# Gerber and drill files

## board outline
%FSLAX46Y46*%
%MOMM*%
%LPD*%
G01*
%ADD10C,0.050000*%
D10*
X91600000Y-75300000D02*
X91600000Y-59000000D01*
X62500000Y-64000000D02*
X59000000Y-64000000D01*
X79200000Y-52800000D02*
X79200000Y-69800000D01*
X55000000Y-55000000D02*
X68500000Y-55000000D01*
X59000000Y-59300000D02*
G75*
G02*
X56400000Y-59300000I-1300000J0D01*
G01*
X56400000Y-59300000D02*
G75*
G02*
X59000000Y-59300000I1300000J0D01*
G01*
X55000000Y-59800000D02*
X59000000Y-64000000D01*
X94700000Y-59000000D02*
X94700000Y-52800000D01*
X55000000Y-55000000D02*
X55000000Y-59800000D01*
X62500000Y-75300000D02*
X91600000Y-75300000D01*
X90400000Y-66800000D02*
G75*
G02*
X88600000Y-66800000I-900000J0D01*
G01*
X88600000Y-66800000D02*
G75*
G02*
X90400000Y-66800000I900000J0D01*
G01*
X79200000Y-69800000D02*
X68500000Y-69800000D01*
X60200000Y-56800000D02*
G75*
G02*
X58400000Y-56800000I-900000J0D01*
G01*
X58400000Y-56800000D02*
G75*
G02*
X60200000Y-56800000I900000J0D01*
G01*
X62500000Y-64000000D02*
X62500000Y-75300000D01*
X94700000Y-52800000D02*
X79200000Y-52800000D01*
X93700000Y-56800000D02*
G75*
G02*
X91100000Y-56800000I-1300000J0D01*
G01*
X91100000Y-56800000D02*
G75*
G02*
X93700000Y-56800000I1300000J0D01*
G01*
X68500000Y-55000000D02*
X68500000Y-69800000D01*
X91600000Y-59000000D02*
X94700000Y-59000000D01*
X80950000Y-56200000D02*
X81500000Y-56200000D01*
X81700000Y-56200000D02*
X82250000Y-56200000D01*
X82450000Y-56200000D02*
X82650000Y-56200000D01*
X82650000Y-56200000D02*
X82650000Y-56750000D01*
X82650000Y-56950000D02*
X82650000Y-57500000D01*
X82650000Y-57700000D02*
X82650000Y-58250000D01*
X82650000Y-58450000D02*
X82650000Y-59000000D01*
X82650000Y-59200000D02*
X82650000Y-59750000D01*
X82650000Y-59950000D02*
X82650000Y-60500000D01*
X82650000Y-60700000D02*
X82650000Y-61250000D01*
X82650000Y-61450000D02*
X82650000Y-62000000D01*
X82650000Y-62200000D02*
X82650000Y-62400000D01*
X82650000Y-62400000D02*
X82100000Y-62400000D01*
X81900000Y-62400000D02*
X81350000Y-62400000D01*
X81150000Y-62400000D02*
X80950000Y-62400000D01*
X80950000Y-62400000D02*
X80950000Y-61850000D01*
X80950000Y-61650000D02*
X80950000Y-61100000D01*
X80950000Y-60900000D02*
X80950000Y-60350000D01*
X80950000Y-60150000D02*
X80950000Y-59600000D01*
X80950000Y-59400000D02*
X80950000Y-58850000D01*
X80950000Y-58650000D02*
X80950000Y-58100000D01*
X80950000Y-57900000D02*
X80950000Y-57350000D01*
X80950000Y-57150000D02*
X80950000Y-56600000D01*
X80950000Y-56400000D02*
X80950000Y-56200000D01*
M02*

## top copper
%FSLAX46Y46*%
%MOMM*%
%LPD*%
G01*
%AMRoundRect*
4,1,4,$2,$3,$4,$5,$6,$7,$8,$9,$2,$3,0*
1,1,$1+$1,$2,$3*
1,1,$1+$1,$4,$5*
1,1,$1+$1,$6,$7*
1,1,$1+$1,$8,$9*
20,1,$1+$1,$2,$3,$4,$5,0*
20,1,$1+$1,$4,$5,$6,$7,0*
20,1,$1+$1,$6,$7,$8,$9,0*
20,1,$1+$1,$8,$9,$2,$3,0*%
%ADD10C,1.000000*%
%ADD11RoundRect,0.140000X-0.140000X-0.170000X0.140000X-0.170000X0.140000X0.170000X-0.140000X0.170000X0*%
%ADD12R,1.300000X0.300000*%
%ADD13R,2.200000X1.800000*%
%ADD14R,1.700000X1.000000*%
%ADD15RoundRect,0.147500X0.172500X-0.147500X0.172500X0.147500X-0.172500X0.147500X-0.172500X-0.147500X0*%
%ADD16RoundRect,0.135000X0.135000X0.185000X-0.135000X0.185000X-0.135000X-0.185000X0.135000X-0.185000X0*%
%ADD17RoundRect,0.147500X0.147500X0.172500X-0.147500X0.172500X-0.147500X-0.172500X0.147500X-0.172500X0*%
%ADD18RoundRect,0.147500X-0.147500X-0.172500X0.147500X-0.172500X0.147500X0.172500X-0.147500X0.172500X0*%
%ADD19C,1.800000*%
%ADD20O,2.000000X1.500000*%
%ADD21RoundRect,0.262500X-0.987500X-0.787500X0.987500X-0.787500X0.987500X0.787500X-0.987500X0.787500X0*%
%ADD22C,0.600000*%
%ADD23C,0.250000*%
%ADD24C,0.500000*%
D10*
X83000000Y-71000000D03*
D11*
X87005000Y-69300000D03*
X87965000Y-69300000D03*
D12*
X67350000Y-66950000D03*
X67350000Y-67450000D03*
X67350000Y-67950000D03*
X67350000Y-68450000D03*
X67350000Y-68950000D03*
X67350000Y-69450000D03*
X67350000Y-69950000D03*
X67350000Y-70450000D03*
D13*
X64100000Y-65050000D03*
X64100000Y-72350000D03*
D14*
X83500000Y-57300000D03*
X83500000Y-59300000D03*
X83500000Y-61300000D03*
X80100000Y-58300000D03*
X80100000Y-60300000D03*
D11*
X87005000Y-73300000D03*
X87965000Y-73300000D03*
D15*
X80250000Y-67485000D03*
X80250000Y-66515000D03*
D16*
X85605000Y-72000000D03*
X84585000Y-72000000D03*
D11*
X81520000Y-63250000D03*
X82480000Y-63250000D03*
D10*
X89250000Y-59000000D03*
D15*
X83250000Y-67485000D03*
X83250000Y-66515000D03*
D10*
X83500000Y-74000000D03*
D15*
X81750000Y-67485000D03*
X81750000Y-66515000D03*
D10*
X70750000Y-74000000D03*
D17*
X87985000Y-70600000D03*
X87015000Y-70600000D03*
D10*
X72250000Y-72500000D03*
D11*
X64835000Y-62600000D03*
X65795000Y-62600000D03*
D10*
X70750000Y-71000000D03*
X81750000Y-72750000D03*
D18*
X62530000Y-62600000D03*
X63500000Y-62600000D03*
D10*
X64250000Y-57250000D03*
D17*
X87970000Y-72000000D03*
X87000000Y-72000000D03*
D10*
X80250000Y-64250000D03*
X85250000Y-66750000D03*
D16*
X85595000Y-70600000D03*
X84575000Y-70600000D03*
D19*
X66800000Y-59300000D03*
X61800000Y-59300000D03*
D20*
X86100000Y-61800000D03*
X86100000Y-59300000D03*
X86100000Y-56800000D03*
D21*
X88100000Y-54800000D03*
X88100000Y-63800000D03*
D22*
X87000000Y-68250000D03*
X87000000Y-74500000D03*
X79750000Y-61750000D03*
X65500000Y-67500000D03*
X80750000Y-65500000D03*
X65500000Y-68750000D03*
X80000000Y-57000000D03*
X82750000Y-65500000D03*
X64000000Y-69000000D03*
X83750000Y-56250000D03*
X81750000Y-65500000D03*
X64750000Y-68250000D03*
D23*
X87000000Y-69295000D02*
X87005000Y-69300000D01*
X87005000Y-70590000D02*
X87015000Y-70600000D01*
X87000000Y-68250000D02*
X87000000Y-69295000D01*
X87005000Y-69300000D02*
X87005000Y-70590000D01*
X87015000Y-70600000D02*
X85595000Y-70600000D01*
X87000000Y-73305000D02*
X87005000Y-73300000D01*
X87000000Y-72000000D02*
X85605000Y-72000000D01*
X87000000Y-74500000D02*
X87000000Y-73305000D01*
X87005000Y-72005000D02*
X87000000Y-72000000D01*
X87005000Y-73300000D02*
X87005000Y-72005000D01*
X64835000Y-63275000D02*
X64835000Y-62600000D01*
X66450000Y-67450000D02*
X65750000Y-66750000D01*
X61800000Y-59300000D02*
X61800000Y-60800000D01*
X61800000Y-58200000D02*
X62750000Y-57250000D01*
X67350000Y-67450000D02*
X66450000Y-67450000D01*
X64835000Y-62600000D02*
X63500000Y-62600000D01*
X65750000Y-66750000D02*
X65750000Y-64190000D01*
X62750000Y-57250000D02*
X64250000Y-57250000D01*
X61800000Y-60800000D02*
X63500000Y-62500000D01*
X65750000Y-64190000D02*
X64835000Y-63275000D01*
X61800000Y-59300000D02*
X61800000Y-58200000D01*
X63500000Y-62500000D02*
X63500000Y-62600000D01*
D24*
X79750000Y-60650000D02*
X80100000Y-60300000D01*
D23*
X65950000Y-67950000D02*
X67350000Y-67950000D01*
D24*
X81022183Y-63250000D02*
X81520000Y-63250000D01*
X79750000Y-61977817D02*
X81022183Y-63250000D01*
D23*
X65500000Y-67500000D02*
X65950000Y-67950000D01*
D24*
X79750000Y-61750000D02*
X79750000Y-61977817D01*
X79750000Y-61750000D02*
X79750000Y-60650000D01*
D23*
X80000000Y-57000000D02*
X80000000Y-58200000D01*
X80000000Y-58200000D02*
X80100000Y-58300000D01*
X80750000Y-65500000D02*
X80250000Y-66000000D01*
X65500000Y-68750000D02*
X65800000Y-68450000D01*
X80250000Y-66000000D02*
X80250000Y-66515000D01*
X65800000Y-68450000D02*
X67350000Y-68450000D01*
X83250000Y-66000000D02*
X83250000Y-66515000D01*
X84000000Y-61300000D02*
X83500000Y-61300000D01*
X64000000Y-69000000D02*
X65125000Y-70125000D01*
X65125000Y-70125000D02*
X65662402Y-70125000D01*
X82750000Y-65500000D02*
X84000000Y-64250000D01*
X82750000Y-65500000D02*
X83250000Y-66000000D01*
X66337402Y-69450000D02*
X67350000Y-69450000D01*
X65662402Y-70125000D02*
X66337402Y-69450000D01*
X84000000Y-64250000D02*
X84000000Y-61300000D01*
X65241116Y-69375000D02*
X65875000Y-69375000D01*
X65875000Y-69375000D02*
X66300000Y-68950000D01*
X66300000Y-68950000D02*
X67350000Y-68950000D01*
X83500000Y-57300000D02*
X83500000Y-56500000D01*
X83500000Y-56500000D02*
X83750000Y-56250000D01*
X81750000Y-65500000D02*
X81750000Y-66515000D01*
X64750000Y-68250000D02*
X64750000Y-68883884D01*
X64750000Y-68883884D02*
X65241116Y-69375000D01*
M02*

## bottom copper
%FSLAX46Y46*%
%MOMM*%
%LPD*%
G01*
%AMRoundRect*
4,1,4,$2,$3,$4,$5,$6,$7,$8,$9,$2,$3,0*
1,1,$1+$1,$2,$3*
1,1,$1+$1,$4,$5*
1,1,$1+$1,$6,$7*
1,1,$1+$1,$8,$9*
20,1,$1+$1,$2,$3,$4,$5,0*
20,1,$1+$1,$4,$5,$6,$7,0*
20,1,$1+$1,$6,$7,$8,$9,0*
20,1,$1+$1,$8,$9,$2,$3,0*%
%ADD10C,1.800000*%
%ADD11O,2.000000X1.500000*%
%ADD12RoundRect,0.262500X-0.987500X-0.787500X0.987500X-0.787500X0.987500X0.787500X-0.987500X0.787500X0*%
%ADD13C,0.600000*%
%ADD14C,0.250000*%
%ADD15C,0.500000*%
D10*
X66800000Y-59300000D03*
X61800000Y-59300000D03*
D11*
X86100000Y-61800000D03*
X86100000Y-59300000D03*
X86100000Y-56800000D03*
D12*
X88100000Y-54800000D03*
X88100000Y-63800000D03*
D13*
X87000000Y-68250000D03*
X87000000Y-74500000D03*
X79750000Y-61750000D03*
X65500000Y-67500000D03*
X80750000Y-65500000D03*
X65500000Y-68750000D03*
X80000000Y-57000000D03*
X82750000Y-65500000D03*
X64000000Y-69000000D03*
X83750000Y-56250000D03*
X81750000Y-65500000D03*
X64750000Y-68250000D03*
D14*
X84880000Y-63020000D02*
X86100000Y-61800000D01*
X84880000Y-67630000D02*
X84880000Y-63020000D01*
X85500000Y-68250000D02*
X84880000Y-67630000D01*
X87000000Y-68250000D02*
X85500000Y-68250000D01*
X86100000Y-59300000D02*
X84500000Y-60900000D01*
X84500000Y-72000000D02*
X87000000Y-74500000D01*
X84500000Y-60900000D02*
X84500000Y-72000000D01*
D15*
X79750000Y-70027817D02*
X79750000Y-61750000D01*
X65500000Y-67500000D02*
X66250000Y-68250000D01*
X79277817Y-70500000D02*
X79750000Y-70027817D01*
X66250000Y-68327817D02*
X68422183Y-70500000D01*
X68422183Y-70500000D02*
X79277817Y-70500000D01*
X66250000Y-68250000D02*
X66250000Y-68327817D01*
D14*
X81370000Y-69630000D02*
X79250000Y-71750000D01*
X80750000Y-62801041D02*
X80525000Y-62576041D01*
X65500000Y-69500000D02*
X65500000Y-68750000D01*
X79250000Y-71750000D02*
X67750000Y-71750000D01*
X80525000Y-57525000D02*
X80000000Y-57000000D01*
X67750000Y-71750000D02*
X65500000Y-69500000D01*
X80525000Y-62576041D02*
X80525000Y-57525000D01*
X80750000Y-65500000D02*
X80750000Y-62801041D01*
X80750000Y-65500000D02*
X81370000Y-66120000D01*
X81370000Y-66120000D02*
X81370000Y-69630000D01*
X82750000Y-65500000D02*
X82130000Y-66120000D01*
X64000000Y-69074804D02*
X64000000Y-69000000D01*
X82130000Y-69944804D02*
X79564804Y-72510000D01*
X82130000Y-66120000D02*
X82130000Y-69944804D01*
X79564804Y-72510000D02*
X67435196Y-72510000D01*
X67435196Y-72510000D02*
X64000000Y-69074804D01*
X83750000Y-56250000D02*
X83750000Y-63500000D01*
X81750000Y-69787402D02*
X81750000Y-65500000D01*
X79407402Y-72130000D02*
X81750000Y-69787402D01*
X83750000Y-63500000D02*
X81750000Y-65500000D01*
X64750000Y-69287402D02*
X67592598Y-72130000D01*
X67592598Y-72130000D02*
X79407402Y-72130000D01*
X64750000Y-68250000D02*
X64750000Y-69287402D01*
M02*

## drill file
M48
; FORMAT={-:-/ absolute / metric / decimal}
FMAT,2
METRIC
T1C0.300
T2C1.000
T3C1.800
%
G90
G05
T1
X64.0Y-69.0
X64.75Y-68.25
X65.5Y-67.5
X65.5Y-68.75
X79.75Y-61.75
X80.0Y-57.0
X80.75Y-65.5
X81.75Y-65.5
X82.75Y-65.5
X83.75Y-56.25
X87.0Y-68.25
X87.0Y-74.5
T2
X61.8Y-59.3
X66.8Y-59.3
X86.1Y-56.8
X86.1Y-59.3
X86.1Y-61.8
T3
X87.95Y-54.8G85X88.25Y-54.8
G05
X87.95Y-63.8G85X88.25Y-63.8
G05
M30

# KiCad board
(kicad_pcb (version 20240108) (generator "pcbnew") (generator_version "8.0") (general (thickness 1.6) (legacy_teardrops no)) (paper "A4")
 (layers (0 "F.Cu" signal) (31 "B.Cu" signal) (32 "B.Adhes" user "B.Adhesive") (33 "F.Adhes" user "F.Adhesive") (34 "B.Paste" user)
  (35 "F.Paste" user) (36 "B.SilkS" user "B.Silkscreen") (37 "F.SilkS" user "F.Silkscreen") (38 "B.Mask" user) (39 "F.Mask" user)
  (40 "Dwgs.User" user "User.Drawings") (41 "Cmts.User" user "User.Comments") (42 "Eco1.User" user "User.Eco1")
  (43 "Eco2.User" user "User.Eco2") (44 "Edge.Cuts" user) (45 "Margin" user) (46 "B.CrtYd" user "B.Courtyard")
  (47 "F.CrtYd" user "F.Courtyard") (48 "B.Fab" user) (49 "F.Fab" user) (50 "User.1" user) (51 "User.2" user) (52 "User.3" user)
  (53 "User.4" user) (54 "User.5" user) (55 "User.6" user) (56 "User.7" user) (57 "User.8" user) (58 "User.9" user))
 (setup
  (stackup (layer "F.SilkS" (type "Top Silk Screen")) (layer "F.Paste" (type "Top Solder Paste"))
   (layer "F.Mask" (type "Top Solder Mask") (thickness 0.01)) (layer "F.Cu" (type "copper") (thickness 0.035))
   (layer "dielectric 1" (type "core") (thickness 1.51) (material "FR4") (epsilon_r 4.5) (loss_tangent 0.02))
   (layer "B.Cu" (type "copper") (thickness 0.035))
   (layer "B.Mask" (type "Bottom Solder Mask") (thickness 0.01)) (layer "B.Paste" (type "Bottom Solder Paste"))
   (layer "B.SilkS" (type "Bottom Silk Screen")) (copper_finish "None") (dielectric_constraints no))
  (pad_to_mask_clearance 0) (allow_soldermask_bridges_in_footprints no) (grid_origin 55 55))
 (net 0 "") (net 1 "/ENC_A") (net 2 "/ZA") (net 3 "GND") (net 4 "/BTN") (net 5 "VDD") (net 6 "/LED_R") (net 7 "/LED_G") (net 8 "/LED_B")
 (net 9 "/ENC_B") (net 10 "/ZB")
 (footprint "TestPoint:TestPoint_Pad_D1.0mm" (layer "F.Cu") (at 83 71)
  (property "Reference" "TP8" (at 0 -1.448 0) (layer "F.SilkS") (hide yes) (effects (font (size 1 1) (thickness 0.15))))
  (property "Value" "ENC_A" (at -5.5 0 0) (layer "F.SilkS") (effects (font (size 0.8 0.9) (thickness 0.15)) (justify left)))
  (pad "1" smd circle (at 0 0) (size 1 1) (layers "F.Cu" "F.Mask") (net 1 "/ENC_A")))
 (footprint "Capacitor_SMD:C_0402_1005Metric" (layer "F.Cu") (at 87.485 69.3)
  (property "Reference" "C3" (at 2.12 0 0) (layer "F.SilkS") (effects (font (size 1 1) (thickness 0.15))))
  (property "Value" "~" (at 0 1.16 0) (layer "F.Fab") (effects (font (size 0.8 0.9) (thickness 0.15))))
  (pad "1" smd roundrect (at -0.48 0) (size 0.56 0.62) (layers "F.Cu" "F.Paste" "F.Mask") (roundrect_rratio 0.25) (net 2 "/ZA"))
  (pad "2" smd roundrect (at 0.48 0) (size 0.56 0.62) (layers "F.Cu" "F.Paste" "F.Mask") (roundrect_rratio 0.25) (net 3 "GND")))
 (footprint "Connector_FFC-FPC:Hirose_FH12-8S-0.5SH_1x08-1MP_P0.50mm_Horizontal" (layer "F.Cu") (at 65.5 68.7 -90)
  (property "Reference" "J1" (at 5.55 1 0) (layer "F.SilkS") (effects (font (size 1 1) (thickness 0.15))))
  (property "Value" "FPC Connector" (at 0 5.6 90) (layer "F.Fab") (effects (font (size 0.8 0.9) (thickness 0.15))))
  (pad "1" smd rect (at -1.75 -1.85 270) (size 0.3 1.3) (layers "F.Cu" "F.Paste" "F.Mask") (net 3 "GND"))
  (pad "2" smd rect (at -1.25 -1.85 270) (size 0.3 1.3) (layers "F.Cu" "F.Paste" "F.Mask") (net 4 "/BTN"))
  (pad "3" smd rect (at -0.75 -1.85 270) (size 0.3 1.3) (layers "F.Cu" "F.Paste" "F.Mask") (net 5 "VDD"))
  (pad "4" smd rect (at -0.25 -1.85 270) (size 0.3 1.3) (layers "F.Cu" "F.Paste" "F.Mask") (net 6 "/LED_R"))
  (pad "5" smd rect (at 0.25 -1.85 270) (size 0.3 1.3) (layers "F.Cu" "F.Paste" "F.Mask") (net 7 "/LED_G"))
  (pad "6" smd rect (at 0.75 -1.85 270) (size 0.3 1.3) (layers "F.Cu" "F.Paste" "F.Mask") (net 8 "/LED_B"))
  (pad "7" smd rect (at 1.25 -1.85 270) (size 0.3 1.3) (layers "F.Cu" "F.Paste" "F.Mask") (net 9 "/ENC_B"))
  (pad "8" smd rect (at 1.75 -1.85 270) (size 0.3 1.3) (layers "F.Cu" "F.Paste" "F.Mask") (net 1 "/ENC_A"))
  (pad "MP" smd rect (at -3.65 1.4 270) (size 1.8 2.2) (layers "F.Cu" "F.Paste" "F.Mask") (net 3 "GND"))
  (pad "MP" smd rect (at 3.65 1.4 270) (size 1.8 2.2) (layers "F.Cu" "F.Paste" "F.Mask") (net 3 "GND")))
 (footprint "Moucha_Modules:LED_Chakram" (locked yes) (layer "F.Cu") (at 81.8 59.3)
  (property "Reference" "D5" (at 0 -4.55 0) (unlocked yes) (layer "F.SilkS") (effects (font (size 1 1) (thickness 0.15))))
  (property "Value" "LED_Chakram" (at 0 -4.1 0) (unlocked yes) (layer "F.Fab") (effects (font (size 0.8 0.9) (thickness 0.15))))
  (fp_rect (start -0.85 -3.1) (end 0.85 3.1) (stroke (width 0.05) (type dash)) (fill none) (layer "Edge.Cuts"))
  (pad "1" smd rect (at 1.7 -2) (size 1.7 1) (layers "F.Cu" "F.Paste" "F.Mask") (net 7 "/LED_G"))
  (pad "2" smd rect (at 1.7 0) (size 1.7 1) (layers "F.Cu" "F.Paste" "F.Mask") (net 3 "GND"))
  (pad "3" smd rect (at 1.7 2) (size 1.7 1) (layers "F.Cu" "F.Paste" "F.Mask") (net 8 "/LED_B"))
  (pad "4" smd rect (at -1.7 -1) (size 1.7 1) (layers "F.Cu" "F.Paste" "F.Mask") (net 6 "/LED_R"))
  (pad "5" smd rect (at -1.7 1) (size 1.7 1) (layers "F.Cu" "F.Paste" "F.Mask") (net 5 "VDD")))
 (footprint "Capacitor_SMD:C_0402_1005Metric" (layer "F.Cu") (at 87.485 73.3)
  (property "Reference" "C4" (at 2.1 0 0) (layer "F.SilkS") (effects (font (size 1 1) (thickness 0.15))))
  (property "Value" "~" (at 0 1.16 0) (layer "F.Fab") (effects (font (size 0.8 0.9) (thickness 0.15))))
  (pad "1" smd roundrect (at -0.48 0) (size 0.56 0.62) (layers "F.Cu" "F.Paste" "F.Mask") (roundrect_rratio 0.25) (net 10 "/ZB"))
  (pad "2" smd roundrect (at 0.48 0) (size 0.56 0.62) (layers "F.Cu" "F.Paste" "F.Mask") (roundrect_rratio 0.25) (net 3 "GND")))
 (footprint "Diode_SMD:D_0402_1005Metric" (layer "F.Cu") (at 80.25 67 90)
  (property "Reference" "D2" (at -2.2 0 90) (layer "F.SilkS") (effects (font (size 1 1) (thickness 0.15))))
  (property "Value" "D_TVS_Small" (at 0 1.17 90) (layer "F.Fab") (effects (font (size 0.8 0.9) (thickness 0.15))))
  (pad "1" smd roundrect (at -0.485 0 90) (size 0.59 0.64) (layers "F.Cu" "F.Paste" "F.Mask") (roundrect_rratio 0.25) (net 3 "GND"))
  (pad "2" smd roundrect (at 0.485 0 90) (size 0.59 0.64) (layers "F.Cu" "F.Paste" "F.Mask") (roundrect_rratio 0.25) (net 6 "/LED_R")))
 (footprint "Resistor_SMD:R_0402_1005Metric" (layer "F.Cu") (at 85.095 72 180)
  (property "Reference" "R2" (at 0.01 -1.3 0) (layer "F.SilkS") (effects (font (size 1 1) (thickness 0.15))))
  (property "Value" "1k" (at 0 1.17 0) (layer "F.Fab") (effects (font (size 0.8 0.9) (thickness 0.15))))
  (pad "1" smd roundrect (at -0.51 0 180) (size 0.54 0.64) (layers "F.Cu" "F.Paste" "F.Mask") (roundrect_rratio 0.25) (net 10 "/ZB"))
  (pad "2" smd roundrect (at 0.51 0 180) (size 0.54 0.64) (layers "F.Cu" "F.Paste" "F.Mask") (roundrect_rratio 0.25) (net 9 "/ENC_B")))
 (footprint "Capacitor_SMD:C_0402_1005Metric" (layer "F.Cu") (at 82 63.25)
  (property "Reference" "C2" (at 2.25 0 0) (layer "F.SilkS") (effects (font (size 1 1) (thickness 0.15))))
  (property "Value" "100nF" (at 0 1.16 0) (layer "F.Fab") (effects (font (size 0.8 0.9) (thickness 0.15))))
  (pad "1" smd roundrect (at -0.48 0) (size 0.56 0.62) (layers "F.Cu" "F.Paste" "F.Mask") (roundrect_rratio 0.25) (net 5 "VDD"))
  (pad "2" smd roundrect (at 0.48 0) (size 0.56 0.62) (layers "F.Cu" "F.Paste" "F.Mask") (roundrect_rratio 0.25) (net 3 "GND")))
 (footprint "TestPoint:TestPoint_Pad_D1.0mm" (layer "F.Cu") (at 89.25 59)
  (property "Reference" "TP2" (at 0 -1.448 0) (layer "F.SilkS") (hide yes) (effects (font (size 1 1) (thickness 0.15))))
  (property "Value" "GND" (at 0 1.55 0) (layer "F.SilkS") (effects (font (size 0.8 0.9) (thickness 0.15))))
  (pad "1" smd circle (at 0 0) (size 1 1) (layers "F.Cu" "F.Mask") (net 3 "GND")))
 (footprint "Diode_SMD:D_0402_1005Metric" (layer "F.Cu") (at 83.25 67 90)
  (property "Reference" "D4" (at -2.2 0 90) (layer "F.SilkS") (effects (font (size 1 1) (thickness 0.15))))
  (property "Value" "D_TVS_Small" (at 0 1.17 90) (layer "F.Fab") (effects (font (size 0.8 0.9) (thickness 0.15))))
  (pad "1" smd roundrect (at -0.485 0 90) (size 0.59 0.64) (layers "F.Cu" "F.Paste" "F.Mask") (roundrect_rratio 0.25) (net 3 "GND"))
  (pad "2" smd roundrect (at 0.485 0 90) (size 0.59 0.64) (layers "F.Cu" "F.Paste" "F.Mask") (roundrect_rratio 0.25) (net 8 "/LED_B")))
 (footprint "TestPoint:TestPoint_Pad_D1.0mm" (layer "F.Cu") (at 83.5 74)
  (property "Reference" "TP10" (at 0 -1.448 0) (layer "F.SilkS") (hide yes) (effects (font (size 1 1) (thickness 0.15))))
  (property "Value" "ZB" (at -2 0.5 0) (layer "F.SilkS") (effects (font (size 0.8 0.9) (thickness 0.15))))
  (pad "1" smd circle (at 0 0) (size 1 1) (layers "F.Cu" "F.Mask") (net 10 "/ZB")))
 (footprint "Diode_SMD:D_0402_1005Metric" (layer "F.Cu") (at 81.75 67 90)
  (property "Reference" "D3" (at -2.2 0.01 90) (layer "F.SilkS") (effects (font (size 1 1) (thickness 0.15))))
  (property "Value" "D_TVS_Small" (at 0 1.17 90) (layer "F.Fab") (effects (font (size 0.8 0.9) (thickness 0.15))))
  (pad "1" smd roundrect (at -0.485 0 90) (size 0.59 0.64) (layers "F.Cu" "F.Paste" "F.Mask") (roundrect_rratio 0.25) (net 3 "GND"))
  (pad "2" smd roundrect (at 0.485 0 90) (size 0.59 0.64) (layers "F.Cu" "F.Paste" "F.Mask") (roundrect_rratio 0.25) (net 7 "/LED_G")))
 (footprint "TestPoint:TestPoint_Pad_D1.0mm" (layer "F.Cu") (at 70.75 74)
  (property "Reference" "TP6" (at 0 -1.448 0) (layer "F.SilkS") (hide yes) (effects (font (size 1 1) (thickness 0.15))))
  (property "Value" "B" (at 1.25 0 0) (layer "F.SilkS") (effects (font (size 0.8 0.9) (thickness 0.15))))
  (pad "1" smd circle (at 0 0) (size 1 1) (layers "F.Cu" "F.Mask") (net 8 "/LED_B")))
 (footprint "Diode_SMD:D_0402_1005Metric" (layer "F.Cu") (at 87.5 70.6 180)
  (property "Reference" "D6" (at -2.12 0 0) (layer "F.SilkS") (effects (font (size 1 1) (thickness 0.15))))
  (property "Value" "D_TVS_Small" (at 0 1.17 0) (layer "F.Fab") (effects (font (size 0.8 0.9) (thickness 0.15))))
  (pad "1" smd roundrect (at -0.485 0 180) (size 0.59 0.64) (layers "F.Cu" "F.Paste" "F.Mask") (roundrect_rratio 0.25) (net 3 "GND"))
  (pad "2" smd roundrect (at 0.485 0 180) (size 0.59 0.64) (layers "F.Cu" "F.Paste" "F.Mask") (roundrect_rratio 0.25) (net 2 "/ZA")))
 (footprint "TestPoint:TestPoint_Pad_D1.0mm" (layer "F.Cu") (at 72.25 72.5)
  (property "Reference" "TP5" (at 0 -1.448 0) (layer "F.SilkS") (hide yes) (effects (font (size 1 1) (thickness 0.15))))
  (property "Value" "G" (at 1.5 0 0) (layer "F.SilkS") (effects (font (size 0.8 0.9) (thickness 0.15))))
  (pad "1" smd circle (at 0 0) (size 1 1) (layers "F.Cu" "F.Mask") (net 7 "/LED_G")))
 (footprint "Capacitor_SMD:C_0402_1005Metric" (layer "F.Cu") (at 65.315 62.6)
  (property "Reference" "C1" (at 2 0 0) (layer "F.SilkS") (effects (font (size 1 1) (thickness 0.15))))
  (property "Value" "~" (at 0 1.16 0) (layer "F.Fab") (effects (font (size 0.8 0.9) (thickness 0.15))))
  (pad "1" smd roundrect (at -0.48 0) (size 0.56 0.62) (layers "F.Cu" "F.Paste" "F.Mask") (roundrect_rratio 0.25) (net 4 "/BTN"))
  (pad "2" smd roundrect (at 0.48 0) (size 0.56 0.62) (layers "F.Cu" "F.Paste" "F.Mask") (roundrect_rratio 0.25) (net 3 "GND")))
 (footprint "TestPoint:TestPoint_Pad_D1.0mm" (layer "F.Cu") (at 70.75 71)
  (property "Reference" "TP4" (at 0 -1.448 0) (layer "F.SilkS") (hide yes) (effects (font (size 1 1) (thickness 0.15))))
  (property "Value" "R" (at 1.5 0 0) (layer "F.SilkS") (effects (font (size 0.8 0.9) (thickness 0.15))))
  (pad "1" smd circle (at 0 0) (size 1 1) (layers "F.Cu" "F.Mask") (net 6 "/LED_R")))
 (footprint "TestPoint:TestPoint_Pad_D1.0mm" (layer "F.Cu") (at 81.75 72.75)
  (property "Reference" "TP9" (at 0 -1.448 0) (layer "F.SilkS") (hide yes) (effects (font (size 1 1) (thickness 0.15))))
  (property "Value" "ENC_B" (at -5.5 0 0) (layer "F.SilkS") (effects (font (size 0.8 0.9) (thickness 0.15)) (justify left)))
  (pad "1" smd circle (at 0 0) (size 1 1) (layers "F.Cu" "F.Mask") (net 9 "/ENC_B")))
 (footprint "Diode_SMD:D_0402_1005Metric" (layer "F.Cu") (at 63.015 62.6)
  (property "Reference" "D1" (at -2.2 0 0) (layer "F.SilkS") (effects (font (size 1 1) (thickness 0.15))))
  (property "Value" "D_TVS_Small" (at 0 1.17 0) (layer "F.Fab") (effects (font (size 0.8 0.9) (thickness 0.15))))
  (pad "1" smd roundrect (at -0.485 0) (size 0.59 0.64) (layers "F.Cu" "F.Paste" "F.Mask") (roundrect_rratio 0.25) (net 3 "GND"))
  (pad "2" smd roundrect (at 0.485 0) (size 0.59 0.64) (layers "F.Cu" "F.Paste" "F.Mask") (roundrect_rratio 0.25) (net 4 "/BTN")))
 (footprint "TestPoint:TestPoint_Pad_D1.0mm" (layer "F.Cu") (at 64.25 57.25)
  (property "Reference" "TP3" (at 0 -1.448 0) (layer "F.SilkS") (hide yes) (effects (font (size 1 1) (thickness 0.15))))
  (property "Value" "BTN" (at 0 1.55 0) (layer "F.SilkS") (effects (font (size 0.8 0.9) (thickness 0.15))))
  (pad "1" smd circle (at 0 0) (size 1 1) (layers "F.Cu" "F.Mask") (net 4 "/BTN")))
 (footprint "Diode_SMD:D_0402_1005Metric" (layer "F.Cu") (at 87.485 72 180)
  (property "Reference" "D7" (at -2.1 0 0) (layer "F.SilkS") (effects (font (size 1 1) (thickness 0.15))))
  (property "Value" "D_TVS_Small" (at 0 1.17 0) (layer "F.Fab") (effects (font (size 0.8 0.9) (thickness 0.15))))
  (pad "1" smd roundrect (at -0.485 0 180) (size 0.59 0.64) (layers "F.Cu" "F.Paste" "F.Mask") (roundrect_rratio 0.25) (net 3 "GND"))
  (pad "2" smd roundrect (at 0.485 0 180) (size 0.59 0.64) (layers "F.Cu" "F.Paste" "F.Mask") (roundrect_rratio 0.25) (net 10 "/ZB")))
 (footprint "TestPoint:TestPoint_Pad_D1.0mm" (layer "F.Cu") (at 80.25 64.25)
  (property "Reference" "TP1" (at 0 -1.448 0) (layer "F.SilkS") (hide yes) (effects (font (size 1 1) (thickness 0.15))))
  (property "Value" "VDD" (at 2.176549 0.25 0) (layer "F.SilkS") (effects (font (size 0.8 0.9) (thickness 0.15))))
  (pad "1" smd circle (at 0 0) (size 1 1) (layers "F.Cu" "F.Mask") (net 5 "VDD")))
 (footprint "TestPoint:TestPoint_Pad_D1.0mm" (layer "F.Cu") (at 85.25 66.75)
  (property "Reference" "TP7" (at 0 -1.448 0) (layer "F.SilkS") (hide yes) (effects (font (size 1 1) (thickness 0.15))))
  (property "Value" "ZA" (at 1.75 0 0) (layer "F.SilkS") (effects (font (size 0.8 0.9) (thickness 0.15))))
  (pad "1" smd circle (at 0 0) (size 1 1) (layers "F.Cu" "F.Mask") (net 2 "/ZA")))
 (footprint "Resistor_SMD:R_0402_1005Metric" (layer "F.Cu") (at 85.085 70.6 180)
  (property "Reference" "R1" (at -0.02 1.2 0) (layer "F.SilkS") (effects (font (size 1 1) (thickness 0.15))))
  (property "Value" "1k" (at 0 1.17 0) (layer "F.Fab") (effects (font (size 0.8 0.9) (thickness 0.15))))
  (pad "1" smd roundrect (at -0.51 0 180) (size 0.54 0.64) (layers "F.Cu" "F.Paste" "F.Mask") (roundrect_rratio 0.25) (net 2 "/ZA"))
  (pad "2" smd roundrect (at 0.51 0 180) (size 0.54 0.64) (layers "F.Cu" "F.Paste" "F.Mask") (roundrect_rratio 0.25) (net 1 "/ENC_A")))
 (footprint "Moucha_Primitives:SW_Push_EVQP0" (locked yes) (layer "B.Cu") (at 64.3 59.3 180)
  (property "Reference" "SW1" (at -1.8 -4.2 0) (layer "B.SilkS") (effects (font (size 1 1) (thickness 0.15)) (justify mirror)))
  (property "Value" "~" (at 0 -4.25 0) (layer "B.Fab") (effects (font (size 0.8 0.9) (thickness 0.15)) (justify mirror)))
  (pad "1" thru_hole circle (at -2.5 0 180) (size 1.8 1.8) (drill 1) (layers "*.Cu" "*.Mask") (remove_unused_layers no) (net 3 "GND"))
  (pad "2" thru_hole circle (at 2.5 0 180) (size 1.8 1.8) (drill 1) (layers "*.Cu" "*.Mask") (remove_unused_layers no) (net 4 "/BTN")))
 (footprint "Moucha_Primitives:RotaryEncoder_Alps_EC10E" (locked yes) (layer "B.Cu") (at 86.1 61.8)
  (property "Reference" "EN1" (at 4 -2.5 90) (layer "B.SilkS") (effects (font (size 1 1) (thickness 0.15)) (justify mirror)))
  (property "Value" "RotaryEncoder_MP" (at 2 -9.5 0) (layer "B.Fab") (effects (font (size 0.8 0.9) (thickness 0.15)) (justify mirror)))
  (pad "A" thru_hole oval (at 0 0) (size 2 1.5) (drill 1) (layers "*.Cu" "*.Mask") (remove_unused_layers no) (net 2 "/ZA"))
  (pad "B" thru_hole oval (at 0 -2.5) (size 2 1.5) (drill 1) (layers "*.Cu" "*.Mask") (remove_unused_layers no) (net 10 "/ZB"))
  (pad "C" thru_hole oval (at 0 -5) (size 2 1.5) (drill 1) (layers "*.Cu" "*.Mask") (remove_unused_layers no) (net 3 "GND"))
  (pad "MP" thru_hole roundrect (at 2 -7) (size 2.5 2.1) (drill oval 2.1 1.8) (layers "*.Cu" "*.Mask") (remove_unused_layers no)
   (roundrect_rratio 0.125) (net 3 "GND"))
  (pad "MP" thru_hole roundrect (at 2 2) (size 2.5 2.1) (drill oval 2.1 1.8) (layers "*.Cu" "*.Mask") (remove_unused_layers no)
   (roundrect_rratio 0.125) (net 3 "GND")))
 (gr_line (start 91.6 75.3) (end 91.6 59) (stroke (width 0.05) (type default)) (layer "Edge.Cuts"))
 (gr_line (start 62.5 64) (end 59 64) (stroke (width 0.05) (type default)) (layer "Edge.Cuts"))
 (gr_line (start 79.2 52.8) (end 79.2 69.8) (stroke (width 0.05) (type default)) (layer "Edge.Cuts"))
 (gr_line (start 55 55) (end 68.5 55) (stroke (width 0.05) (type default)) (layer "Edge.Cuts"))
 (gr_circle (center 57.7 59.3) (end 59 59.3) (stroke (width 0.05) (type default)) (fill none) (layer "Edge.Cuts"))
 (gr_line (start 55 59.8) (end 59 64) (stroke (width 0.05) (type default)) (layer "Edge.Cuts"))
 (gr_line (start 94.7 59) (end 94.7 52.8) (stroke (width 0.05) (type default)) (layer "Edge.Cuts"))
 (gr_line (start 55 55) (end 55 59.8) (stroke (width 0.05) (type default)) (layer "Edge.Cuts"))
 (gr_line (start 62.5 75.3) (end 91.6 75.3) (stroke (width 0.05) (type default)) (layer "Edge.Cuts"))
 (gr_circle (center 89.5 66.8) (end 90.4 66.8) (stroke (width 0.05) (type default)) (fill none) (layer "Edge.Cuts"))
 (gr_line (start 79.2 69.8) (end 68.5 69.8) (stroke (width 0.05) (type default)) (layer "Edge.Cuts"))
 (gr_circle (center 59.3 56.8) (end 60.2 56.8) (stroke (width 0.05) (type default)) (fill none) (layer "Edge.Cuts"))
 (gr_line (start 62.5 64) (end 62.5 75.3) (stroke (width 0.05) (type default)) (layer "Edge.Cuts"))
 (gr_line (start 94.7 52.8) (end 79.2 52.8) (stroke (width 0.05) (type default)) (layer "Edge.Cuts"))
 (gr_circle (center 92.4 56.8) (end 93.7 56.8) (stroke (width 0.05) (type default)) (fill none) (layer "Edge.Cuts"))
 (gr_line (start 68.5 55) (end 68.5 69.8) (stroke (width 0.05) (type default)) (layer "Edge.Cuts"))
 (gr_line (start 91.6 59) (end 94.7 59) (stroke (width 0.05) (type default)) (layer "Edge.Cuts"))
 (segment (start 87 69.295) (end 87.005 69.3) (width 0.25) (layer "F.Cu") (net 2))
 (segment (start 87.005 70.59) (end 87.015 70.6) (width 0.25) (layer "F.Cu") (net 2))
 (segment (start 87 68.25) (end 87 69.295) (width 0.25) (layer "F.Cu") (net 2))
 (segment (start 87.005 69.3) (end 87.005 70.59) (width 0.25) (layer "F.Cu") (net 2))
 (segment (start 87.015 70.6) (end 85.595 70.6) (width 0.25) (layer "F.Cu") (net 2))
 (via (at 87 68.25) (size 0.6) (drill 0.3) (layers "F.Cu" "B.Cu") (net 2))
 (segment (start 84.88 63.02) (end 86.1 61.8) (width 0.25) (layer "B.Cu") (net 2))
 (segment (start 84.88 67.63) (end 84.88 63.02) (width 0.25) (layer "B.Cu") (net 2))
 (segment (start 85.5 68.25) (end 84.88 67.63) (width 0.25) (layer "B.Cu") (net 2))
 (segment (start 87 68.25) (end 85.5 68.25) (width 0.25) (layer "B.Cu") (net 2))
 (segment (start 87 73.305) (end 87.005 73.3) (width 0.25) (layer "F.Cu") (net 10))
 (segment (start 87 72) (end 85.605 72) (width 0.25) (layer "F.Cu") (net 10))
 (segment (start 87 74.5) (end 87 73.305) (width 0.25) (layer "F.Cu") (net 10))
 (segment (start 87.005 72.005) (end 87 72) (width 0.25) (layer "F.Cu") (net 10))
 (segment (start 87.005 73.3) (end 87.005 72.005) (width 0.25) (layer "F.Cu") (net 10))
 (via (at 87 74.5) (size 0.6) (drill 0.3) (layers "F.Cu" "B.Cu") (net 10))
 (segment (start 86.1 59.3) (end 84.5 60.9) (width 0.25) (layer "B.Cu") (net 10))
 (segment (start 84.5 72) (end 87 74.5) (width 0.25) (layer "B.Cu") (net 10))
 (segment (start 84.5 60.9) (end 84.5 72) (width 0.25) (layer "B.Cu") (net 10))
 (segment (start 64.835 63.275) (end 64.835 62.6) (width 0.25) (layer "F.Cu") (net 4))
 (segment (start 66.45 67.45) (end 65.75 66.75) (width 0.25) (layer "F.Cu") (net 4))
 (segment (start 61.8 59.3) (end 61.8 60.8) (width 0.25) (layer "F.Cu") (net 4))
 (segment (start 61.8 58.2) (end 62.75 57.25) (width 0.25) (layer "F.Cu") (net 4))
 (segment (start 67.35 67.45) (end 66.45 67.45) (width 0.25) (layer "F.Cu") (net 4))
 (segment (start 64.835 62.6) (end 63.5 62.6) (width 0.25) (layer "F.Cu") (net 4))
 (segment (start 65.75 66.75) (end 65.75 64.19) (width 0.25) (layer "F.Cu") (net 4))
 (segment (start 62.75 57.25) (end 64.25 57.25) (width 0.25) (layer "F.Cu") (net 4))
 (segment (start 61.8 60.8) (end 63.5 62.5) (width 0.25) (layer "F.Cu") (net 4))
 (segment (start 65.75 64.19) (end 64.835 63.275) (width 0.25) (layer "F.Cu") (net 4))
 (segment (start 61.8 59.3) (end 61.8 58.2) (width 0.25) (layer "F.Cu") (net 4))
 (segment (start 63.5 62.5) (end 63.5 62.6) (width 0.25) (layer "F.Cu") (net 4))
 (segment (start 79.75 60.65) (end 80.1 60.3) (width 0.5) (layer "F.Cu") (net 5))
 (segment (start 65.95 67.95) (end 67.35 67.95) (width 0.25) (layer "F.Cu") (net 5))
 (segment (start 81.022183 63.25) (end 81.52 63.25) (width 0.5) (layer "F.Cu") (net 5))
 (segment (start 79.75 61.977817) (end 81.022183 63.25) (width 0.5) (layer "F.Cu") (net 5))
 (segment (start 65.5 67.5) (end 65.95 67.95) (width 0.25) (layer "F.Cu") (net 5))
 (segment (start 79.75 61.75) (end 79.75 61.977817) (width 0.5) (layer "F.Cu") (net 5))
 (segment (start 79.75 61.75) (end 79.75 60.65) (width 0.5) (layer "F.Cu") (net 5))
 (via (at 79.75 61.75) (size 0.6) (drill 0.3) (layers "F.Cu" "B.Cu") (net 5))
 (via (at 65.5 67.5) (size 0.6) (drill 0.3) (layers "F.Cu" "B.Cu") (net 5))
 (segment (start 79.75 70.027817) (end 79.75 61.75) (width 0.5) (layer "B.Cu") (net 5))
 (segment (start 65.5 67.5) (end 66.25 68.25) (width 0.5) (layer "B.Cu") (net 5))
 (segment (start 79.277817 70.5) (end 79.75 70.027817) (width 0.5) (layer "B.Cu") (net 5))
 (segment (start 66.25 68.327817) (end 68.422183 70.5) (width 0.5) (layer "B.Cu") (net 5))
 (segment (start 68.422183 70.5) (end 79.277817 70.5) (width 0.5) (layer "B.Cu") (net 5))
 (segment (start 66.25 68.25) (end 66.25 68.327817) (width 0.5) (layer "B.Cu") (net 5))
 (segment (start 80 57) (end 80 58.2) (width 0.25) (layer "F.Cu") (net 6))
 (segment (start 80 58.2) (end 80.1 58.3) (width 0.25) (layer "F.Cu") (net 6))
 (segment (start 80.75 65.5) (end 80.25 66) (width 0.25) (layer "F.Cu") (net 6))
 (segment (start 65.5 68.75) (end 65.8 68.45) (width 0.25) (layer "F.Cu") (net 6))
 (segment (start 80.25 66) (end 80.25 66.515) (width 0.25) (layer "F.Cu") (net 6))
 (segment (start 65.8 68.45) (end 67.35 68.45) (width 0.25) (layer "F.Cu") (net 6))
 (via (at 80.75 65.5) (size 0.6) (drill 0.3) (layers "F.Cu" "B.Cu") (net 6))
 (via (at 65.5 68.75) (size 0.6) (drill 0.3) (layers "F.Cu" "B.Cu") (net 6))
 (via (at 80 57) (size 0.6) (drill 0.3) (layers "F.Cu" "B.Cu") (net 6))
 (segment (start 81.37 69.63) (end 79.25 71.75) (width 0.25) (layer "B.Cu") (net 6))
 (segment (start 80.75 62.801041) (end 80.525 62.576041) (width 0.25) (layer "B.Cu") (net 6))
 (segment (start 65.5 69.5) (end 65.5 68.75) (width 0.25) (layer "B.Cu") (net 6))
 (segment (start 79.25 71.75) (end 67.75 71.75) (width 0.25) (layer "B.Cu") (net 6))
 (segment (start 80.525 57.525) (end 80 57) (width 0.25) (layer "B.Cu") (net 6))
 (segment (start 67.75 71.75) (end 65.5 69.5) (width 0.25) (layer "B.Cu") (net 6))
 (segment (start 80.525 62.576041) (end 80.525 57.525) (width 0.25) (layer "B.Cu") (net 6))
 (segment (start 80.75 65.5) (end 80.75 62.801041) (width 0.25) (layer "B.Cu") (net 6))
 (segment (start 80.75 65.5) (end 81.37 66.12) (width 0.25) (layer "B.Cu") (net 6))
 (segment (start 81.37 66.12) (end 81.37 69.63) (width 0.25) (layer "B.Cu") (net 6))
 (segment (start 83.25 66) (end 83.25 66.515) (width 0.25) (layer "F.Cu") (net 8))
 (segment (start 84 61.3) (end 83.5 61.3) (width 0.25) (layer "F.Cu") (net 8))
 (segment (start 64 69) (end 65.125 70.125) (width 0.25) (layer "F.Cu") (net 8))
 (segment (start 65.125 70.125) (end 65.662402 70.125) (width 0.25) (layer "F.Cu") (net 8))
 (segment (start 82.75 65.5) (end 84 64.25) (width 0.25) (layer "F.Cu") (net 8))
 (segment (start 82.75 65.5) (end 83.25 66) (width 0.25) (layer "F.Cu") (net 8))
 (segment (start 66.337402 69.45) (end 67.35 69.45) (width 0.25) (layer "F.Cu") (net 8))
 (segment (start 65.662402 70.125) (end 66.337402 69.45) (width 0.25) (layer "F.Cu") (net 8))
 (segment (start 84 64.25) (end 84 61.3) (width 0.25) (layer "F.Cu") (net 8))
 (via (at 82.75 65.5) (size 0.6) (drill 0.3) (layers "F.Cu" "B.Cu") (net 8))
 (via (at 64 69) (size 0.6) (drill 0.3) (layers "F.Cu" "B.Cu") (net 8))
 (segment (start 82.75 65.5) (end 82.13 66.12) (width 0.25) (layer "B.Cu") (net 8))
 (segment (start 64 69.074804) (end 64 69) (width 0.25) (layer "B.Cu") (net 8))
 (segment (start 82.13 69.944804) (end 79.564804 72.51) (width 0.25) (layer "B.Cu") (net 8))
 (segment (start 82.13 66.12) (end 82.13 69.944804) (width 0.25) (layer "B.Cu") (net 8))
 (segment (start 79.564804 72.51) (end 67.435196 72.51) (width 0.25) (layer "B.Cu") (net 8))
 (segment (start 67.435196 72.51) (end 64 69.074804) (width 0.25) (layer "B.Cu") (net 8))
 (segment (start 65.241116 69.375) (end 65.875 69.375) (width 0.25) (layer "F.Cu") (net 7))
 (segment (start 65.875 69.375) (end 66.3 68.95) (width 0.25) (layer "F.Cu") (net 7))
 (segment (start 66.3 68.95) (end 67.35 68.95) (width 0.25) (layer "F.Cu") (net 7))
 (segment (start 83.5 57.3) (end 83.5 56.5) (width 0.25) (layer "F.Cu") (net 7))
 (segment (start 83.5 56.5) (end 83.75 56.25) (width 0.25) (layer "F.Cu") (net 7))
 (segment (start 81.75 65.5) (end 81.75 66.515) (width 0.25) (layer "F.Cu") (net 7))
 (segment (start 64.75 68.25) (end 64.75 68.883884) (width 0.25) (layer "F.Cu") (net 7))
 (segment (start 64.75 68.883884) (end 65.241116 69.375) (width 0.25) (layer "F.Cu") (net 7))
 (via (at 83.75 56.25) (size 0.6) (drill 0.3) (layers "F.Cu" "B.Cu") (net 7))
 (via (at 81.75 65.5) (size 0.6) (drill 0.3) (layers "F.Cu" "B.Cu") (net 7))
 (via (at 64.75 68.25) (size 0.6) (drill 0.3) (layers "F.Cu" "B.Cu") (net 7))
 (segment (start 83.75 56.25) (end 83.75 63.5) (width 0.25) (layer "B.Cu") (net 7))
 (segment (start 81.75 69.787402) (end 81.75 65.5) (width 0.25) (layer "B.Cu") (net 7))
 (segment (start 79.407402 72.13) (end 81.75 69.787402) (width 0.25) (layer "B.Cu") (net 7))
 (segment (start 83.75 63.5) (end 81.75 65.5) (width 0.25) (layer "B.Cu") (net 7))
 (segment (start 64.75 69.287402) (end 67.592598 72.13) (width 0.25) (layer "B.Cu") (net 7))
 (segment (start 67.592598 72.13) (end 79.407402 72.13) (width 0.25) (layer "B.Cu") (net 7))
 (segment (start 64.75 68.25) (end 64.75 69.287402) (width 0.25) (layer "B.Cu") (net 7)))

